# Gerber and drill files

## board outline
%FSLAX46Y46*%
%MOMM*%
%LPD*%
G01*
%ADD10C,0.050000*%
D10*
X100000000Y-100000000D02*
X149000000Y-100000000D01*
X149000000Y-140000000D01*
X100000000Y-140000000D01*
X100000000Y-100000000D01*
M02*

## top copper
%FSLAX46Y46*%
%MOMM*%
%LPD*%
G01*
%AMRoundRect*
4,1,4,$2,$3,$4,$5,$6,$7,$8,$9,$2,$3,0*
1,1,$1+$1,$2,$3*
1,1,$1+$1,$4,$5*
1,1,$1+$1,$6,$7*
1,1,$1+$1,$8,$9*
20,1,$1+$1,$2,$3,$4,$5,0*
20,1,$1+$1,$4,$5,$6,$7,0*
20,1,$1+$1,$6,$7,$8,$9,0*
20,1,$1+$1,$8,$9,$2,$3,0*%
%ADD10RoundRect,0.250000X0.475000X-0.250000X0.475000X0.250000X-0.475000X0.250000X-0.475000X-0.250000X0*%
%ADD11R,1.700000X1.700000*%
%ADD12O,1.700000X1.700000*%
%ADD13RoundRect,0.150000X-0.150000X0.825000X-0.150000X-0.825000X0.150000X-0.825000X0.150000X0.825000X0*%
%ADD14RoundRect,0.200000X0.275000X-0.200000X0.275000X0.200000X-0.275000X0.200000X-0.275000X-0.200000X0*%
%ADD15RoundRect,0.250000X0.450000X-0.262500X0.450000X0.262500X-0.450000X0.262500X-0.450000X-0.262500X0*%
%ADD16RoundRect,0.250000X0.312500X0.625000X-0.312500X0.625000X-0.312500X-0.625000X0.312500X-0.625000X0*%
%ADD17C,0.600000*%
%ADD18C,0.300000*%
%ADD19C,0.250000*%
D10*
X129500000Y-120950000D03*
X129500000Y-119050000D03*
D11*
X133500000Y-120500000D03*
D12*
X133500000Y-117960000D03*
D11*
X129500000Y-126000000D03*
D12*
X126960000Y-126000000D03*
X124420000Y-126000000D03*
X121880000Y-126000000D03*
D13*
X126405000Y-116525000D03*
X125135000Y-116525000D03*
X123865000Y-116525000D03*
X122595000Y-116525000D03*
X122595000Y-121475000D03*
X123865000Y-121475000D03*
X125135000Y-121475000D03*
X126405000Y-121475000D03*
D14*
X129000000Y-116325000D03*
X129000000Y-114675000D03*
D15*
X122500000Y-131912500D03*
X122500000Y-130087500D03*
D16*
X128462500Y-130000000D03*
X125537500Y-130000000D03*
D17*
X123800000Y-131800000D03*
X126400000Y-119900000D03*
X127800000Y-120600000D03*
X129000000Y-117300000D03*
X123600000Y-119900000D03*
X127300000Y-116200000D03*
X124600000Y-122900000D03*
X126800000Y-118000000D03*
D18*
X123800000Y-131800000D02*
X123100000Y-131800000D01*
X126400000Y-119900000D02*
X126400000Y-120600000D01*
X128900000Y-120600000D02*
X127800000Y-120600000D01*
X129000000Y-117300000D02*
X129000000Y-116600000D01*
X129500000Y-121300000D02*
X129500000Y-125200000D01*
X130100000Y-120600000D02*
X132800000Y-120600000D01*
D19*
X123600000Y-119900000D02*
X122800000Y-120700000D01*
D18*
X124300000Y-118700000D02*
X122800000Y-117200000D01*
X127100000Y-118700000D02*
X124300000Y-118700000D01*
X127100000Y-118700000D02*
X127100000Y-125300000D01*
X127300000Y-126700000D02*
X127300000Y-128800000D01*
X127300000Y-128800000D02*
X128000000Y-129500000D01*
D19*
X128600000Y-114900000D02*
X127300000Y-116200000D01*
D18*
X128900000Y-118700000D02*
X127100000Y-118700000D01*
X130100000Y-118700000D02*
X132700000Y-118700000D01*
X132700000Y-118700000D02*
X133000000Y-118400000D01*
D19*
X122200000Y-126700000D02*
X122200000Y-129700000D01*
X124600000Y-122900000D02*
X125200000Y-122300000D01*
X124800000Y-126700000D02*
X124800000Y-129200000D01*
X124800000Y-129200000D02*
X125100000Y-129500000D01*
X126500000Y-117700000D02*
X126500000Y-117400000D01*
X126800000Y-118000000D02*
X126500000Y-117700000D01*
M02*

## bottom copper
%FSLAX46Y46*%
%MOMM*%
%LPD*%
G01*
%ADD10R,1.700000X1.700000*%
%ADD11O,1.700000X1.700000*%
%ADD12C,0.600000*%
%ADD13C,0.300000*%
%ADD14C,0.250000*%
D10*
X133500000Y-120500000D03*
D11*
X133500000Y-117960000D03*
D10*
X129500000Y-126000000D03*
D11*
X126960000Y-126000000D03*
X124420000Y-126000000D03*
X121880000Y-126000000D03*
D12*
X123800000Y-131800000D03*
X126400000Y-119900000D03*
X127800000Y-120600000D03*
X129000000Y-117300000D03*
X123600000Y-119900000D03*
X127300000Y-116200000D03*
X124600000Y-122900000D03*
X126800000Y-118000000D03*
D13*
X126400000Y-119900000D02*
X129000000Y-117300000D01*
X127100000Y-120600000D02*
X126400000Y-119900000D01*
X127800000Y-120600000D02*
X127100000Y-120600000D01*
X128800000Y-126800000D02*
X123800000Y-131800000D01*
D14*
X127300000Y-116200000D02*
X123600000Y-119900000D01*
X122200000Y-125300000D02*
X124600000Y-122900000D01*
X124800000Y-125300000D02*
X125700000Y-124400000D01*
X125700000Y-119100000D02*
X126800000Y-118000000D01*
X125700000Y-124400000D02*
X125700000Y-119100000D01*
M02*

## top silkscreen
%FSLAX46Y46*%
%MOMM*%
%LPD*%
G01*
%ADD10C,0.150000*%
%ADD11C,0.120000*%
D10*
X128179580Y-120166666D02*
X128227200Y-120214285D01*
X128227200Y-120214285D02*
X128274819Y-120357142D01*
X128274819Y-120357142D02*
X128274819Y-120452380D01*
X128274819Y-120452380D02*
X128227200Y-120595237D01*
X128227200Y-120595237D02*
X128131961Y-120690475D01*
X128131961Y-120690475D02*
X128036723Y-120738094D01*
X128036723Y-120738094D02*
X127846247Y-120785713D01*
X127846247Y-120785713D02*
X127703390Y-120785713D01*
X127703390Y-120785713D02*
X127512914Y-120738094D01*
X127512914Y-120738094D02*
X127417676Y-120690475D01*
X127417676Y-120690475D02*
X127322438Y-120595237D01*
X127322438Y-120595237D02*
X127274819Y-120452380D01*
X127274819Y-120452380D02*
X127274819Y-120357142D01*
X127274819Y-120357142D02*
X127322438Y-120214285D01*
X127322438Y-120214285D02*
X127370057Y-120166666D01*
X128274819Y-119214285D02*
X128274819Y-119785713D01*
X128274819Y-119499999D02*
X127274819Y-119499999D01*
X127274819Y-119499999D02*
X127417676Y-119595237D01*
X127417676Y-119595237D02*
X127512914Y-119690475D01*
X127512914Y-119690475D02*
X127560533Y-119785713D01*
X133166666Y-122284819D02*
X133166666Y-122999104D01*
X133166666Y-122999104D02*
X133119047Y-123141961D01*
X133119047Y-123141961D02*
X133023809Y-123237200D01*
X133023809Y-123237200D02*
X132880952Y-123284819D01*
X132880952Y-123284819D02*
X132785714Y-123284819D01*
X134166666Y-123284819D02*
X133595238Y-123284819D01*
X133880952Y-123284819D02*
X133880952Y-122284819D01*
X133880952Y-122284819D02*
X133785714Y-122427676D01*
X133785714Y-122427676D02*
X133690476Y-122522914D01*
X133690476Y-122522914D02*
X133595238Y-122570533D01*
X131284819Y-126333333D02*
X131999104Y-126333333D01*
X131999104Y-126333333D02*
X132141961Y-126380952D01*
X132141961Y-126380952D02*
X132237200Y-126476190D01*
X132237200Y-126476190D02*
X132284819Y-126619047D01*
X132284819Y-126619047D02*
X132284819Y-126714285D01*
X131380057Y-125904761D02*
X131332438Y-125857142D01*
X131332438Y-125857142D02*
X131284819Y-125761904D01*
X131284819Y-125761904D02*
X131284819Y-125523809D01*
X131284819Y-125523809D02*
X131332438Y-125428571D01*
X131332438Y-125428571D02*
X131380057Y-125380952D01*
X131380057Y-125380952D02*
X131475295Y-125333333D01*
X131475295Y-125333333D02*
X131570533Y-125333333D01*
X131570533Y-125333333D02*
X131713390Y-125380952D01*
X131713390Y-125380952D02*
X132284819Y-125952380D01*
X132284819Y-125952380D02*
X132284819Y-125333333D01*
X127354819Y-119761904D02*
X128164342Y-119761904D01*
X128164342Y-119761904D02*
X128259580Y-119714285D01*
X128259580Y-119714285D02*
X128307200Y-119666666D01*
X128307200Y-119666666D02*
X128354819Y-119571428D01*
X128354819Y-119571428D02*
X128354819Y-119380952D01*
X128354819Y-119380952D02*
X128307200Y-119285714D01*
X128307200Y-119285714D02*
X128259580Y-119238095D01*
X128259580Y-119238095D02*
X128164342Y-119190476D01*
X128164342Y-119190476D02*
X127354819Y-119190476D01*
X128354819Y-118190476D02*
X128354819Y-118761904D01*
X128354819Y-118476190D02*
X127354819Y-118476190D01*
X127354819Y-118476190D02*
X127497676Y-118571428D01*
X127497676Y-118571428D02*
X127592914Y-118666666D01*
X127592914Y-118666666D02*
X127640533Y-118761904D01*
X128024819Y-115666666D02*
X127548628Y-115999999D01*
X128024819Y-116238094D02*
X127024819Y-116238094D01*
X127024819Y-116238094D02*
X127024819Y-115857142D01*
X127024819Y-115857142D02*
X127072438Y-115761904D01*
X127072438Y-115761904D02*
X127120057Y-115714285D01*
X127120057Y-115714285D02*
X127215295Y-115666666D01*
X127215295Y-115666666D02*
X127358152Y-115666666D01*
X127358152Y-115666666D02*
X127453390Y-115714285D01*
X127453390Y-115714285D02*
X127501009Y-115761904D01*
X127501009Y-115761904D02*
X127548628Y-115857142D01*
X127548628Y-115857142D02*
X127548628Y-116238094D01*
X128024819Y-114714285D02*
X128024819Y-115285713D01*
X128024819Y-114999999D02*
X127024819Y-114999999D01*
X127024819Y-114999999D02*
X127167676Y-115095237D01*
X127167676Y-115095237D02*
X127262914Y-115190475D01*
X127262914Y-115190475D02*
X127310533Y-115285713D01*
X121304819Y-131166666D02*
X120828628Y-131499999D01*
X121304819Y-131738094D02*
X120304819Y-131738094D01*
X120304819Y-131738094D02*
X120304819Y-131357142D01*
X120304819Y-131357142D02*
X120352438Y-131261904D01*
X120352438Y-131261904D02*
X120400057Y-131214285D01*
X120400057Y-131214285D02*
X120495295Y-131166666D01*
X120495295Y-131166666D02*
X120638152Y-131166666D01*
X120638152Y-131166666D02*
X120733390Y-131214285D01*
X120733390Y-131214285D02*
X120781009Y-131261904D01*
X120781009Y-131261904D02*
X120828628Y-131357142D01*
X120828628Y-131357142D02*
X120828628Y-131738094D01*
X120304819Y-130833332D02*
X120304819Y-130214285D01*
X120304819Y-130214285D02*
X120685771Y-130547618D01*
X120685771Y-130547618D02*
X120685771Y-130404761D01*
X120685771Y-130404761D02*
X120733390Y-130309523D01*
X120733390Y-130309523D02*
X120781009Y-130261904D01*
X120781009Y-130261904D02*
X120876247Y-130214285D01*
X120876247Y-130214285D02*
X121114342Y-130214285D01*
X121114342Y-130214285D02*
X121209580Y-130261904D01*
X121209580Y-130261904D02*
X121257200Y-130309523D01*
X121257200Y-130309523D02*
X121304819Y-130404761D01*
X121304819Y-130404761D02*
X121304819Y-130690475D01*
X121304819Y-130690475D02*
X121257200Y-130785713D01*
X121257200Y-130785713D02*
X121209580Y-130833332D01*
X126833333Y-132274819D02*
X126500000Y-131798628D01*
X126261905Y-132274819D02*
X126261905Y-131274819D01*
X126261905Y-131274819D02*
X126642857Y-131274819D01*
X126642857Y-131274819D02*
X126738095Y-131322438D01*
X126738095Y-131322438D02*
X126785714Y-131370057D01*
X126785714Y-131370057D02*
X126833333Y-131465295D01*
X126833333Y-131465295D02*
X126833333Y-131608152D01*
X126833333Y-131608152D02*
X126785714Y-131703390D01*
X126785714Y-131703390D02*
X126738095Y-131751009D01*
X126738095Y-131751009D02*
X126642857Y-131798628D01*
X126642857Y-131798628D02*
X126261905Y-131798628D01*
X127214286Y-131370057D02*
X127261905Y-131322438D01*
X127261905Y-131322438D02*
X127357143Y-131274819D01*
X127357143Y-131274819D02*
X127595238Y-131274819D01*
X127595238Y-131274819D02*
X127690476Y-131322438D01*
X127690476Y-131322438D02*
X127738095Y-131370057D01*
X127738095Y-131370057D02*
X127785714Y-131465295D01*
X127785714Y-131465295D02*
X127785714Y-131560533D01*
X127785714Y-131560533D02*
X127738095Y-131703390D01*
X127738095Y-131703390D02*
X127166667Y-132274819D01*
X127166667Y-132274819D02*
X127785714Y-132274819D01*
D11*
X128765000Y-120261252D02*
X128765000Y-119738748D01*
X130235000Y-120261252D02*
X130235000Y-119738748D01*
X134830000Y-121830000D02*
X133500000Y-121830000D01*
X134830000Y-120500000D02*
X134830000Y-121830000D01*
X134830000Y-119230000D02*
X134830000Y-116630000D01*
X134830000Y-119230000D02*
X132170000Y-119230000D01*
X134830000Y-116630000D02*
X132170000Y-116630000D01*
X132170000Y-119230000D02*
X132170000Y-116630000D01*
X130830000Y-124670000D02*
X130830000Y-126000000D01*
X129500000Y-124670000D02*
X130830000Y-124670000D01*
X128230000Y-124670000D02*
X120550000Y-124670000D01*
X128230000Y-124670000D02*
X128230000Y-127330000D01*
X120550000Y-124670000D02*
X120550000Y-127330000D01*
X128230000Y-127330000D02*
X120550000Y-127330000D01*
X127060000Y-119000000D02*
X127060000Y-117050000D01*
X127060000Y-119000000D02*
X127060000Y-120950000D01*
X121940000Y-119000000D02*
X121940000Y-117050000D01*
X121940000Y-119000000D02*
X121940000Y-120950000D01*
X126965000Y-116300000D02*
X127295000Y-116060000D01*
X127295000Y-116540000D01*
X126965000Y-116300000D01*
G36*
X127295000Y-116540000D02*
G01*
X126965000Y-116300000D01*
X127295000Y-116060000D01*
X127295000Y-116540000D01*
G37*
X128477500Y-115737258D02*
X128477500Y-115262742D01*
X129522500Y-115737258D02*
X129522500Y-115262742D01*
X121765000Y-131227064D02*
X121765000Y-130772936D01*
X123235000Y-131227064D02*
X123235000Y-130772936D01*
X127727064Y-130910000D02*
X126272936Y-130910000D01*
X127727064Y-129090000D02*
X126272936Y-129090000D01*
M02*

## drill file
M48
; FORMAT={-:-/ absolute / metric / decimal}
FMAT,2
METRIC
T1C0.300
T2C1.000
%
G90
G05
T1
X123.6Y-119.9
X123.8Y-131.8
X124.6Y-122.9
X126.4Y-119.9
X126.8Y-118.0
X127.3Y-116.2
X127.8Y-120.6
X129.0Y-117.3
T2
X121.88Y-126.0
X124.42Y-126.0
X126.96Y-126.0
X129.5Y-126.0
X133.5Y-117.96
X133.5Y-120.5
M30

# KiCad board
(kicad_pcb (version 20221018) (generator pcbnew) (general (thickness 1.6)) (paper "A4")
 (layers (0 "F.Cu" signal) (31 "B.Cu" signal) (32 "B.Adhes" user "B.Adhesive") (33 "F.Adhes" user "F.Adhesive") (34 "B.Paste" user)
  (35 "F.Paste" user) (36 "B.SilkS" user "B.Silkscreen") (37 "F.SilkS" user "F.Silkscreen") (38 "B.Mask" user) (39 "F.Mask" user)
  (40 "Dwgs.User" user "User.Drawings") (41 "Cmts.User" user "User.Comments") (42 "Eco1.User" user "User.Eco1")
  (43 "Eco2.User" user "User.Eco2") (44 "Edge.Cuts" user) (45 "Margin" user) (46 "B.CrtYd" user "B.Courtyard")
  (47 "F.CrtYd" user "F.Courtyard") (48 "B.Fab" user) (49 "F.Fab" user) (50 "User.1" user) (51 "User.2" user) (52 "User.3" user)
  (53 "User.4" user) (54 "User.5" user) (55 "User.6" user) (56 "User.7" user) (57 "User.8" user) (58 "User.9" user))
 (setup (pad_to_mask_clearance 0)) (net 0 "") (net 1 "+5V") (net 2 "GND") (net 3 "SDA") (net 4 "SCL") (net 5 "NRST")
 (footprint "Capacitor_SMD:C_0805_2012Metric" (layer "F.Cu") (at 129.5 120 90)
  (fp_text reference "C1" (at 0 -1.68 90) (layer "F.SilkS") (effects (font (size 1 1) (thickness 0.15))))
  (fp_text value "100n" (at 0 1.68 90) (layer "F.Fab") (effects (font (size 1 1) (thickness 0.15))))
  (fp_line (start -0.261252 -0.735) (end 0.261252 -0.735) (stroke (width 0.12) (type solid)) (layer "F.SilkS"))
  (fp_line (start -0.261252 0.735) (end 0.261252 0.735) (stroke (width 0.12) (type solid)) (layer "F.SilkS"))
  (pad "1" smd roundrect (at -0.95 0 90) (size 1 1.45) (layers "F.Cu" "F.Paste" "F.Mask") (roundrect_rratio 0.25) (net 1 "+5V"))
  (pad "2" smd roundrect (at 0.95 0 90) (size 1 1.45) (layers "F.Cu" "F.Paste" "F.Mask") (roundrect_rratio 0.25) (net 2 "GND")))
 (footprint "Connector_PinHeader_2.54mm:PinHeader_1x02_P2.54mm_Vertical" (layer "F.Cu") (at 133.5 120.5 180)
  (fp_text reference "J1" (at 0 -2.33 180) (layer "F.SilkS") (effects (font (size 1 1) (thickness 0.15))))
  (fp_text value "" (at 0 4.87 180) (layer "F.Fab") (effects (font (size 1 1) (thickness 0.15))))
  (fp_line (start -1.33 -1.33) (end 0 -1.33) (stroke (width 0.12) (type solid)) (layer "F.SilkS"))
  (fp_line (start -1.33 0) (end -1.33 -1.33) (stroke (width 0.12) (type solid)) (layer "F.SilkS"))
  (fp_line (start -1.33 1.27) (end -1.33 3.87) (stroke (width 0.12) (type solid)) (layer "F.SilkS"))
  (fp_line (start -1.33 1.27) (end 1.33 1.27) (stroke (width 0.12) (type solid)) (layer "F.SilkS"))
  (fp_line (start -1.33 3.87) (end 1.33 3.87) (stroke (width 0.12) (type solid)) (layer "F.SilkS"))
  (fp_line (start 1.33 1.27) (end 1.33 3.87) (stroke (width 0.12) (type solid)) (layer "F.SilkS"))
  (pad "1" thru_hole rect (at 0 0 180) (size 1.7 1.7) (drill 1) (layers "*.Cu" "*.Mask") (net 1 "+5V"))
  (pad "2" thru_hole oval (at 0 2.54 180) (size 1.7 1.7) (drill 1) (layers "*.Cu" "*.Mask") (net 2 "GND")))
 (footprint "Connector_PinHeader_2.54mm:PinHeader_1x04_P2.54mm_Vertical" (layer "F.Cu") (at 129.5 126 -90)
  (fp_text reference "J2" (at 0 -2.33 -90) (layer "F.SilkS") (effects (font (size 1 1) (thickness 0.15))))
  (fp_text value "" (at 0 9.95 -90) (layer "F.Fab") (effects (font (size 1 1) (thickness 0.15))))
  (fp_line (start -1.33 -1.33) (end 0 -1.33) (stroke (width 0.12) (type solid)) (layer "F.SilkS"))
  (fp_line (start -1.33 0) (end -1.33 -1.33) (stroke (width 0.12) (type solid)) (layer "F.SilkS"))
  (fp_line (start -1.33 1.27) (end -1.33 8.95) (stroke (width 0.12) (type solid)) (layer "F.SilkS"))
  (fp_line (start -1.33 1.27) (end 1.33 1.27) (stroke (width 0.12) (type solid)) (layer "F.SilkS"))
  (fp_line (start -1.33 8.95) (end 1.33 8.95) (stroke (width 0.12) (type solid)) (layer "F.SilkS"))
  (fp_line (start 1.33 1.27) (end 1.33 8.95) (stroke (width 0.12) (type solid)) (layer "F.SilkS"))
  (pad "1" thru_hole rect (at 0 0 270) (size 1.7 1.7) (drill 1) (layers "*.Cu" "*.Mask") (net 1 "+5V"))
  (pad "2" thru_hole oval (at 0 2.54 270) (size 1.7 1.7) (drill 1) (layers "*.Cu" "*.Mask") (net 2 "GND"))
  (pad "3" thru_hole oval (at 0 5.08 270) (size 1.7 1.7) (drill 1) (layers "*.Cu" "*.Mask") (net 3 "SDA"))
  (pad "4" thru_hole oval (at 0 7.62 270) (size 1.7 1.7) (drill 1) (layers "*.Cu" "*.Mask") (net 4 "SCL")))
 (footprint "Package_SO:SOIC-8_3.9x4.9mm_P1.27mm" (layer "F.Cu") (at 124.5 119 -90)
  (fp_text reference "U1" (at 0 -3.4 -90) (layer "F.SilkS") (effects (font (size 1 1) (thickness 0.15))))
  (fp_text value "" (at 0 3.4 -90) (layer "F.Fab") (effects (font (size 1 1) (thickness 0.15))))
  (fp_line (start 0 -2.56) (end -1.95 -2.56) (stroke (width 0.12) (type solid)) (layer "F.SilkS"))
  (fp_line (start 0 -2.56) (end 1.95 -2.56) (stroke (width 0.12) (type solid)) (layer "F.SilkS"))
  (fp_line (start 0 2.56) (end -1.95 2.56) (stroke (width 0.12) (type solid)) (layer "F.SilkS"))
  (fp_line (start 0 2.56) (end 1.95 2.56) (stroke (width 0.12) (type solid)) (layer "F.SilkS"))
  (fp_poly
   (pts (xy -2.7 -2.465) (xy -2.94 -2.795) (xy -2.46 -2.795) (xy -2.7 -2.465)) (stroke (width 0.12) (type solid)) (fill solid)
   (layer "F.SilkS"))
  (pad "1" smd roundrect (at -2.475 -1.905 270) (size 1.95 0.6) (layers "F.Cu" "F.Paste" "F.Mask") (roundrect_rratio 0.25) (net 3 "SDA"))
  (pad "2" smd roundrect (at -2.475 -0.635 270) (size 1.95 0.6) (layers "F.Cu" "F.Paste" "F.Mask") (roundrect_rratio 0.25))
  (pad "3" smd roundrect (at -2.475 0.635 270) (size 1.95 0.6) (layers "F.Cu" "F.Paste" "F.Mask") (roundrect_rratio 0.25))
  (pad "4" smd roundrect (at -2.475 1.905 270) (size 1.95 0.6) (layers "F.Cu" "F.Paste" "F.Mask") (roundrect_rratio 0.25) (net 2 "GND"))
  (pad "5" smd roundrect (at 2.475 1.905 270) (size 1.95 0.6) (layers "F.Cu" "F.Paste" "F.Mask") (roundrect_rratio 0.25) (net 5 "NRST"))
  (pad "6" smd roundrect (at 2.475 0.635 270) (size 1.95 0.6) (layers "F.Cu" "F.Paste" "F.Mask") (roundrect_rratio 0.25))
  (pad "7" smd roundrect (at 2.475 -0.635 270) (size 1.95 0.6) (layers "F.Cu" "F.Paste" "F.Mask") (roundrect_rratio 0.25) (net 4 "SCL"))
  (pad "8" smd roundrect (at 2.475 -1.905 270) (size 1.95 0.6) (layers "F.Cu" "F.Paste" "F.Mask") (roundrect_rratio 0.25) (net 1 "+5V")))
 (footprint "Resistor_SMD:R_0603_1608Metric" (layer "F.Cu") (at 129 115.5 90)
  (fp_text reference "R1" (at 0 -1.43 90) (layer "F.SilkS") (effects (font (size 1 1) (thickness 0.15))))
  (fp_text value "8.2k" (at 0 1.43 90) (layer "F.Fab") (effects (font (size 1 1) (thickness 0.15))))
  (fp_line (start -0.237258 -0.5225) (end 0.237258 -0.5225) (stroke (width 0.12) (type solid)) (layer "F.SilkS"))
  (fp_line (start -0.237258 0.5225) (end 0.237258 0.5225) (stroke (width 0.12) (type solid)) (layer "F.SilkS"))
  (pad "1" smd roundrect (at -0.825 0 90) (size 0.8 0.95) (layers "F.Cu" "F.Paste" "F.Mask") (roundrect_rratio 0.25) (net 1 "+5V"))
  (pad "2" smd roundrect (at 0.825 0 90) (size 0.8 0.95) (layers "F.Cu" "F.Paste" "F.Mask") (roundrect_rratio 0.25) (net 5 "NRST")))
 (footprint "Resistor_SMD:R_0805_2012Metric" (layer "F.Cu") (at 122.5 131 90)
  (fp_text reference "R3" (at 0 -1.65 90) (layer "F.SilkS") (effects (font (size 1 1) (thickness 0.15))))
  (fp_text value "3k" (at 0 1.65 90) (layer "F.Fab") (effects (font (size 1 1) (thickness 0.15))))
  (fp_line (start -0.227064 -0.735) (end 0.227064 -0.735) (stroke (width 0.12) (type solid)) (layer "F.SilkS"))
  (fp_line (start -0.227064 0.735) (end 0.227064 0.735) (stroke (width 0.12) (type solid)) (layer "F.SilkS"))
  (pad "1" smd roundrect (at -0.9125 0 90) (size 1.025 1.4) (layers "F.Cu" "F.Paste" "F.Mask") (roundrect_rratio 0.243902) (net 1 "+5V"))
  (pad "2" smd roundrect (at 0.9125 0 90) (size 1.025 1.4) (layers "F.Cu" "F.Paste" "F.Mask") (roundrect_rratio 0.243902) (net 4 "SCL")))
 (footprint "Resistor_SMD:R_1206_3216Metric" (layer "F.Cu") (at 127 130 180)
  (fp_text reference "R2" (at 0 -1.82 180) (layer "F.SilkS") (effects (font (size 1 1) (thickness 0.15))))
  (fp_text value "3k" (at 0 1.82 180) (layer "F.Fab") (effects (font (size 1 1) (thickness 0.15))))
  (fp_line (start -0.727064 -0.91) (end 0.727064 -0.91) (stroke (width 0.12) (type solid)) (layer "F.SilkS"))
  (fp_line (start -0.727064 0.91) (end 0.727064 0.91) (stroke (width 0.12) (type solid)) (layer "F.SilkS"))
  (pad "1" smd roundrect (at -1.4625 0 180) (size 1.125 1.75) (layers "F.Cu" "F.Paste" "F.Mask") (roundrect_rratio 0.222222) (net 2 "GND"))
  (pad "2" smd roundrect (at 1.4625 0 180) (size 1.125 1.75) (layers "F.Cu" "F.Paste" "F.Mask") (roundrect_rratio 0.222222) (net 3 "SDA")))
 (gr_rect (start 100 100) (end 149 140) (stroke (width 0.05) (type default)) (fill none) (layer "Edge.Cuts"))
 (segment (start 123.8 131.8) (end 123.1 131.8) (width 0.3) (layer "F.Cu") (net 1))
 (segment (start 126.4 119.9) (end 126.4 120.6) (width 0.3) (layer "F.Cu") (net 1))
 (segment (start 128.9 120.6) (end 127.8 120.6) (width 0.3) (layer "F.Cu") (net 1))
 (segment (start 129 117.3) (end 129 116.6) (width 0.3) (layer "F.Cu") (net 1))
 (segment (start 129.5 121.3) (end 129.5 125.2) (width 0.3) (layer "F.Cu") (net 1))
 (segment (start 130.1 120.6) (end 132.8 120.6) (width 0.3) (layer "F.Cu") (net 1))
 (via (at 123.8 131.8) (size 0.6) (drill 0.3) (layers "F.Cu" "B.Cu") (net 1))
 (via (at 126.4 119.9) (size 0.6) (drill 0.3) (layers "F.Cu" "B.Cu") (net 1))
 (via (at 127.8 120.6) (size 0.6) (drill 0.3) (layers "F.Cu" "B.Cu") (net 1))
 (via (at 129 117.3) (size 0.6) (drill 0.3) (layers "F.Cu" "B.Cu") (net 1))
 (segment (start 123.6 119.9) (end 122.8 120.7) (width 0.25) (layer "F.Cu") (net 5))
 (segment (start 124.3 118.7) (end 122.8 117.2) (width 0.3) (layer "F.Cu") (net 2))
 (segment (start 126.4 119.9) (end 129 117.3) (width 0.3) (layer "B.Cu") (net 1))
 (segment (start 127.1 118.7) (end 124.3 118.7) (width 0.3) (layer "F.Cu") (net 2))
 (segment (start 127.1 118.7) (end 127.1 125.3) (width 0.3) (layer "F.Cu") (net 2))
 (segment (start 127.1 120.6) (end 126.4 119.9) (width 0.3) (layer "B.Cu") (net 1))
 (segment (start 127.3 126.7) (end 127.3 128.8) (width 0.3) (layer "F.Cu") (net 2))
 (segment (start 127.3 128.8) (end 128 129.5) (width 0.3) (layer "F.Cu") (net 2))
 (segment (start 127.8 120.6) (end 127.1 120.6) (width 0.3) (layer "B.Cu") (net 1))
 (segment (start 128.6 114.9) (end 127.3 116.2) (width 0.25) (layer "F.Cu") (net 5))
 (segment (start 128.8 126.8) (end 123.8 131.8) (width 0.3) (layer "B.Cu") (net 1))
 (segment (start 128.9 118.7) (end 127.1 118.7) (width 0.3) (layer "F.Cu") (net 2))
 (segment (start 130.1 118.7) (end 132.7 118.7) (width 0.3) (layer "F.Cu") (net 2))
 (segment (start 132.7 118.7) (end 133 118.4) (width 0.3) (layer "F.Cu") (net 2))
 (via (at 123.6 119.9) (size 0.6) (drill 0.3) (layers "F.Cu" "B.Cu") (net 5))
 (via (at 127.3 116.2) (size 0.6) (drill 0.3) (layers "F.Cu" "B.Cu") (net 5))
 (segment (start 122.2 126.7) (end 122.2 129.7) (width 0.25) (layer "F.Cu") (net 4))
 (segment (start 124.6 122.9) (end 125.2 122.3) (width 0.25) (layer "F.Cu") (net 4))
 (segment (start 127.3 116.2) (end 123.6 119.9) (width 0.25) (layer "B.Cu") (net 5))
 (via (at 124.6 122.9) (size 0.6) (drill 0.3) (layers "F.Cu" "B.Cu") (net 4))
 (segment (start 122.2 125.3) (end 124.6 122.9) (width 0.25) (layer "B.Cu") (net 4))
 (segment (start 124.8 126.7) (end 124.8 129.2) (width 0.25) (layer "F.Cu") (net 3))
 (segment (start 124.8 129.2) (end 125.1 129.5) (width 0.25) (layer "F.Cu") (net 3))
 (segment (start 126.5 117.7) (end 126.5 117.4) (width 0.25) (layer "F.Cu") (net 3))
 (segment (start 126.8 118) (end 126.5 117.7) (width 0.25) (layer "F.Cu") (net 3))
 (via (at 126.8 118) (size 0.6) (drill 0.3) (layers "F.Cu" "B.Cu") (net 3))
 (segment (start 124.8 125.3) (end 125.7 124.4) (width 0.25) (layer "B.Cu") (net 3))
 (segment (start 125.7 119.1) (end 126.8 118) (width 0.25) (layer "B.Cu") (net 3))
 (segment (start 125.7 124.4) (end 125.7 119.1) (width 0.25) (layer "B.Cu") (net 3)))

